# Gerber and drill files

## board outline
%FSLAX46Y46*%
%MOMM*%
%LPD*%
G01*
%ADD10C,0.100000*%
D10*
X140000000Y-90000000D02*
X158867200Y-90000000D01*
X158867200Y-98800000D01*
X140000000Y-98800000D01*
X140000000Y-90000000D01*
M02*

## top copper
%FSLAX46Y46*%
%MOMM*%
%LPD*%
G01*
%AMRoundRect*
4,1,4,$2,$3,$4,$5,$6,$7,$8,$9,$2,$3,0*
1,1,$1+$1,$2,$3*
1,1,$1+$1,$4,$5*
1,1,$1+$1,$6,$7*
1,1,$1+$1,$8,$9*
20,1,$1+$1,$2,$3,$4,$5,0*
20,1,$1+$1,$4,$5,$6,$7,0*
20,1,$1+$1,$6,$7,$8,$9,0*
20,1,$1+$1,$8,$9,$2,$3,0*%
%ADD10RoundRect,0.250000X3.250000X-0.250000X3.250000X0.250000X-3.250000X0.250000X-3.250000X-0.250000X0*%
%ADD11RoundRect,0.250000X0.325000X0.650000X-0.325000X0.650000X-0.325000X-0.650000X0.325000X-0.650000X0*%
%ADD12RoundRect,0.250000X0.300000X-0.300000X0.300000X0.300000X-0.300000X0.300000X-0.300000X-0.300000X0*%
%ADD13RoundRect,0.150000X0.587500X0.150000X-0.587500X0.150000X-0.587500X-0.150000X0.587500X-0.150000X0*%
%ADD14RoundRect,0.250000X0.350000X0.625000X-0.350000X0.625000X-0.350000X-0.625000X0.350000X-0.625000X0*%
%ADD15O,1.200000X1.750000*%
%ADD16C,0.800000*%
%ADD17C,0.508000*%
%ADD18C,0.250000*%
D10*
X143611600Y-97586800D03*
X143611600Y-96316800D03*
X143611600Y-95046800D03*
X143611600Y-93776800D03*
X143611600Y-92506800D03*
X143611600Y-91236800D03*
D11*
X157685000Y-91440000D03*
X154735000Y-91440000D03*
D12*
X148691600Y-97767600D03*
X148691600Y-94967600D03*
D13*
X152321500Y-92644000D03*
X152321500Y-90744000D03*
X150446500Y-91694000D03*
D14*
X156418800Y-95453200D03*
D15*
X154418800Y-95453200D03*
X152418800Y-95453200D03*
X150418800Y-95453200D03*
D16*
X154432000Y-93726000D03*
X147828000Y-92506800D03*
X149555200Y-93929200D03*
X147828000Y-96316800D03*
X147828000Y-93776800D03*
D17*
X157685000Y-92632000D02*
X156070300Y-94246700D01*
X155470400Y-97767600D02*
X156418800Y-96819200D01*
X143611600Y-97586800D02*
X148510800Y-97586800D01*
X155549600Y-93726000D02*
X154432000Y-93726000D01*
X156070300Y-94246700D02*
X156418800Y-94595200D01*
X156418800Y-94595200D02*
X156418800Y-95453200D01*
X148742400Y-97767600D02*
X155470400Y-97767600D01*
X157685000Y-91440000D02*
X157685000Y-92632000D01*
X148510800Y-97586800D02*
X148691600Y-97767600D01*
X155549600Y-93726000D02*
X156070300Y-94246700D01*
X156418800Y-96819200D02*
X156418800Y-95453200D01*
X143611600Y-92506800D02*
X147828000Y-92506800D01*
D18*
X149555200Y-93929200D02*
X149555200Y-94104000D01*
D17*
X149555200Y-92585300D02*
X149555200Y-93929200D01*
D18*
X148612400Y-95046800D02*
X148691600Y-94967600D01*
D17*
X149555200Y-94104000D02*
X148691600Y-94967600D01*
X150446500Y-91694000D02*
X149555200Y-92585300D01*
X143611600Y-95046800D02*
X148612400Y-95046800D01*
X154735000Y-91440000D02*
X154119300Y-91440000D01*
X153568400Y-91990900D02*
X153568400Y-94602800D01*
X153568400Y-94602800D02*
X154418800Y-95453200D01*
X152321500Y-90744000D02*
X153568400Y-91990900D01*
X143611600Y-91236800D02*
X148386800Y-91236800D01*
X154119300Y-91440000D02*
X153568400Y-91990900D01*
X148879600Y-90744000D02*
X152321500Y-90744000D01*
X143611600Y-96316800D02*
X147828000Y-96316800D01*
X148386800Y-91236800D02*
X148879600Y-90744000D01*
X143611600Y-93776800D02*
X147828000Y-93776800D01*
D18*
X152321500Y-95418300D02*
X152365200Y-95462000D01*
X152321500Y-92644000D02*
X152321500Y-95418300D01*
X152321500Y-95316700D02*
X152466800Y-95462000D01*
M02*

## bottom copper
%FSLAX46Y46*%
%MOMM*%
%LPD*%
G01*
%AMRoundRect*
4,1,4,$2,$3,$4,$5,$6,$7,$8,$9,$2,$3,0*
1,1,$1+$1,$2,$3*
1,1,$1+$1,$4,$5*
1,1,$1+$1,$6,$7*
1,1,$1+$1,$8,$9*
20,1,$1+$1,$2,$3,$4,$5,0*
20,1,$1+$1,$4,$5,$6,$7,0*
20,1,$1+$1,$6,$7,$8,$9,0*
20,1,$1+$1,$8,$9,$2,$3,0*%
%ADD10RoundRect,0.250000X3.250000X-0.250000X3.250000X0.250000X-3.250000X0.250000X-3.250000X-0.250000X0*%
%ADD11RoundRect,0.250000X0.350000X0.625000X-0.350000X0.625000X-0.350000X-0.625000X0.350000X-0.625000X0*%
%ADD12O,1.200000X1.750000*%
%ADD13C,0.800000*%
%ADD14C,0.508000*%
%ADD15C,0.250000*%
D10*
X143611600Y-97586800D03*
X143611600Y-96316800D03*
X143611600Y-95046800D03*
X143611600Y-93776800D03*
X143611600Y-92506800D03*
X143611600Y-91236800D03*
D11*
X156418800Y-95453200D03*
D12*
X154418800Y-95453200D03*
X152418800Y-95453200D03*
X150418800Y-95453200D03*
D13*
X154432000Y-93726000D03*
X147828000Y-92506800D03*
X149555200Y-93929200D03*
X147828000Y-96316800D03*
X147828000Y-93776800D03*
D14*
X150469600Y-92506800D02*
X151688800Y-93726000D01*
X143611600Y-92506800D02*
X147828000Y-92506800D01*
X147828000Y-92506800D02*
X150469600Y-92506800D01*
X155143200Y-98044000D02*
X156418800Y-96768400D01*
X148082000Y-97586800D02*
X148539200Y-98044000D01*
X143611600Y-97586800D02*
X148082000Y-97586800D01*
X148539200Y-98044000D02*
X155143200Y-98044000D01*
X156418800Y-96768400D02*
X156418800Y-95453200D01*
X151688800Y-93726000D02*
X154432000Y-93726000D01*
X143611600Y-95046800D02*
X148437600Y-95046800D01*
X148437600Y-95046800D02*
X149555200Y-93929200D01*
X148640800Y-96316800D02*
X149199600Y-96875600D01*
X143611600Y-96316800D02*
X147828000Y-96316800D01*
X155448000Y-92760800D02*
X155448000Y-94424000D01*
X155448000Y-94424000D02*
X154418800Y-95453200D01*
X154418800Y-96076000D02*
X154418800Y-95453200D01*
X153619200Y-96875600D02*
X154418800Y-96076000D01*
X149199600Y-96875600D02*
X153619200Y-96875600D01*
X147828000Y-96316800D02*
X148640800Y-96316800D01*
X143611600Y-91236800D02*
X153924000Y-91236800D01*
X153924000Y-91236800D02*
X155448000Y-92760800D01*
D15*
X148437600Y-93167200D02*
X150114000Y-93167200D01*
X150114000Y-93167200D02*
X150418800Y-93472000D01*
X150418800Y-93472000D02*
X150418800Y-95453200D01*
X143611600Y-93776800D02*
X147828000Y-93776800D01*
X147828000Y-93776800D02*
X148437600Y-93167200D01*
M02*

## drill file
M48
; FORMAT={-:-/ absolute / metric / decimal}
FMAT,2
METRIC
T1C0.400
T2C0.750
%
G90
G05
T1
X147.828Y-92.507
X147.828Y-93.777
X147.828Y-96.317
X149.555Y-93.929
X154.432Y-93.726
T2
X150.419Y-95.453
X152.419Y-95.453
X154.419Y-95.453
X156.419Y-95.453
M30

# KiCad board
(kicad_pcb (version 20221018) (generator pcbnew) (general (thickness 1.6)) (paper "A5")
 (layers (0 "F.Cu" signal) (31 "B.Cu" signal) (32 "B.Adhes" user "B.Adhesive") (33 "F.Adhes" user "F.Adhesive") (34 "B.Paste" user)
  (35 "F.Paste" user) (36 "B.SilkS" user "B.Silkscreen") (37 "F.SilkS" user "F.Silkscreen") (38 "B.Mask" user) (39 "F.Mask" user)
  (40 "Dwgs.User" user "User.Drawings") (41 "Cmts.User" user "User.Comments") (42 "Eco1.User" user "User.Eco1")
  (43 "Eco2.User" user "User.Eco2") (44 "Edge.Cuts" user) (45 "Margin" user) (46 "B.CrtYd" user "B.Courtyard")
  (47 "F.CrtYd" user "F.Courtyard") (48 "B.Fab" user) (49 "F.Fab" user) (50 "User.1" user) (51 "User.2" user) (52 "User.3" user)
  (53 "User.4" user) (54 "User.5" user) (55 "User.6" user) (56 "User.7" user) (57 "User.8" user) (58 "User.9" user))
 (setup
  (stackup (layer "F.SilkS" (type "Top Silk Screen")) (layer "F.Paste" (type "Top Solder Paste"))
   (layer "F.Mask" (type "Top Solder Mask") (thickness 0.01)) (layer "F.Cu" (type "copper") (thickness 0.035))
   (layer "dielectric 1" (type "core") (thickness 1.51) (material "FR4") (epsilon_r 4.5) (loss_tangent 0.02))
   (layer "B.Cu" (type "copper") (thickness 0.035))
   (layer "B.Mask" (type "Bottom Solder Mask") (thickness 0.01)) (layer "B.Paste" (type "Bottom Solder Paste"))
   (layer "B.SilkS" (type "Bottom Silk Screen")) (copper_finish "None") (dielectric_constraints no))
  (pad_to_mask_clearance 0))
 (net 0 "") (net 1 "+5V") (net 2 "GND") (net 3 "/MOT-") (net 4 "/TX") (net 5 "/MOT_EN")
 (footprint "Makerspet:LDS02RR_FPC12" (layer "F.Cu") (at 143.6116 94.4118 90)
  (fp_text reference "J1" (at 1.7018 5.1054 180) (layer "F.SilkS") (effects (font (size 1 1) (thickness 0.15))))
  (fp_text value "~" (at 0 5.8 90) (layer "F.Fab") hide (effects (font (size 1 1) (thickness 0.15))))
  (pad "1" smd roundrect (at -3.175 0 90) (size 1 7) (layers "F.Cu" "F.Mask") (roundrect_rratio 0.25) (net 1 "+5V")
   (thermal_bridge_angle 45))
  (pad "2" smd roundrect (at -3.175 0 90) (size 1 7) (layers "B.Cu" "B.Mask") (roundrect_rratio 0.25) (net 1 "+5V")
   (thermal_bridge_angle 45))
  (pad "3" smd roundrect (at -1.905 0 90) (size 1 7) (layers "F.Cu" "F.Mask") (roundrect_rratio 0.25) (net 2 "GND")
   (thermal_bridge_angle 45))
  (pad "4" smd roundrect (at -1.905 0 90) (size 1 7) (layers "B.Cu" "B.Mask") (roundrect_rratio 0.25) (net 2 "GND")
   (thermal_bridge_angle 45))
  (pad "5" smd roundrect (at -0.635 0 90) (size 1 7) (layers "F.Cu" "F.Mask") (roundrect_rratio 0.25) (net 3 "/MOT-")
   (thermal_bridge_angle 45))
  (pad "6" smd roundrect (at -0.635 0 90) (size 1 7) (layers "B.Cu" "B.Mask") (roundrect_rratio 0.25) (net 3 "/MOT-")
   (thermal_bridge_angle 45))
  (pad "7" smd roundrect (at 0.635 0 90) (size 1 7) (layers "F.Cu" "F.Mask") (roundrect_rratio 0.25) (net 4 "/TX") (thermal_bridge_angle 45))
  (pad "8" smd roundrect (at 0.635 0 90) (size 1 7) (layers "B.Cu" "B.Mask") (roundrect_rratio 0.25) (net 4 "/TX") (thermal_bridge_angle 45))
  (pad "9" smd roundrect (at 1.905 0 90) (size 1 7) (layers "F.Cu" "F.Mask") (roundrect_rratio 0.25) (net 1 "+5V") (thermal_bridge_angle 45))
  (pad "10" smd roundrect (at 1.905 0 90) (size 1 7) (layers "B.Cu" "B.Mask") (roundrect_rratio 0.25) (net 1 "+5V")
   (thermal_bridge_angle 45))
  (pad "11" smd roundrect (at 3.175 0 90) (size 1 7) (layers "F.Cu" "F.Mask") (roundrect_rratio 0.25) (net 2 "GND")
   (thermal_bridge_angle 45))
  (pad "12" smd roundrect (at 3.175 0 90) (size 1 7) (layers "B.Cu" "B.Mask") (roundrect_rratio 0.25) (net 2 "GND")
   (thermal_bridge_angle 45)))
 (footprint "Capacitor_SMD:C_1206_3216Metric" (layer "F.Cu") (at 156.21 91.44 180)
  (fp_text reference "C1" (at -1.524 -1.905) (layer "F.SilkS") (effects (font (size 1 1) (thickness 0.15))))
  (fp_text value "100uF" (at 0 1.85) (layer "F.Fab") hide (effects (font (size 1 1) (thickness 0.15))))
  (pad "1" smd roundrect (at -1.475 0 180) (size 1.15 1.8) (layers "F.Cu" "F.Paste" "F.Mask") (roundrect_rratio 0.2173913043) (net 1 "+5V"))
  (pad "2" smd roundrect (at 1.475 0 180) (size 1.15 1.8) (layers "F.Cu" "F.Paste" "F.Mask") (roundrect_rratio 0.2173913043) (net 2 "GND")))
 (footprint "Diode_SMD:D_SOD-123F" (layer "F.Cu") (at 148.6916 96.3676 90)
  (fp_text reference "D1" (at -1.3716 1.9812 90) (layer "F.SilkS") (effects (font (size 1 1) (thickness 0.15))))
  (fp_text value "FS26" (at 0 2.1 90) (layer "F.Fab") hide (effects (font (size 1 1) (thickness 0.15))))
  (pad "1" smd roundrect (at -1.4 0 90) (size 1.1 1.1) (layers "F.Cu" "F.Paste" "F.Mask") (roundrect_rratio 0.2272727273) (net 1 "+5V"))
  (pad "2" smd roundrect (at 1.4 0 90) (size 1.1 1.1) (layers "F.Cu" "F.Paste" "F.Mask") (roundrect_rratio 0.2272727273) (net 3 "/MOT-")))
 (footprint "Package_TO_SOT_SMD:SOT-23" (layer "F.Cu") (at 151.384 91.694 180)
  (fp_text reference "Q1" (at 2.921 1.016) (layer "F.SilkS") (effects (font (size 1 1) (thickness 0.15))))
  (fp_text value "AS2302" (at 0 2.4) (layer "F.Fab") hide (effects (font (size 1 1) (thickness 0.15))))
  (pad "1" smd roundrect (at -0.9375 -0.95 180) (size 1.475 0.6) (layers "F.Cu" "F.Paste" "F.Mask") (roundrect_rratio 0.25)
   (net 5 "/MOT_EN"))
  (pad "2" smd roundrect (at -0.9375 0.95 180) (size 1.475 0.6) (layers "F.Cu" "F.Paste" "F.Mask") (roundrect_rratio 0.25) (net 2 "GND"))
  (pad "3" smd roundrect (at 0.9375 0 180) (size 1.475 0.6) (layers "F.Cu" "F.Paste" "F.Mask") (roundrect_rratio 0.25) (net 3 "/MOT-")))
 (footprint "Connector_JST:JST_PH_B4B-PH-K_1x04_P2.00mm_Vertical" (layer "B.Cu") (at 156.4188 95.4532 180)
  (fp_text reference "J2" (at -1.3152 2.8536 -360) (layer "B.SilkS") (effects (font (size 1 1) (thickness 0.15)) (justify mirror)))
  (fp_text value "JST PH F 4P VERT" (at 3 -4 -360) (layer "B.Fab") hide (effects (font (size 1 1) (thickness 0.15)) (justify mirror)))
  (pad "1" thru_hole roundrect (at 0 0 180) (size 1.2 1.75) (drill 0.75) (layers "*.Cu" "*.Mask") (roundrect_rratio 0.2083333333)
   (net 1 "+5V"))
  (pad "2" thru_hole oval (at 2 0 180) (size 1.2 1.75) (drill 0.75) (layers "*.Cu" "*.Mask") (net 2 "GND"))
  (pad "3" thru_hole oval (at 4 0 180) (size 1.2 1.75) (drill 0.75) (layers "*.Cu" "*.Mask") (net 5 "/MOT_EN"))
  (pad "4" thru_hole oval (at 6 0 180) (size 1.2 1.75) (drill 0.75) (layers "*.Cu" "*.Mask") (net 4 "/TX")))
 (gr_rect (start 140 90) (end 158.8672 98.8) (stroke (width 0.1) (type default)) (fill none) (layer "Edge.Cuts"))
 (segment (start 157.685 92.632) (end 156.0703 94.2467) (width 0.508) (layer "F.Cu") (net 1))
 (segment (start 155.4704 97.7676) (end 156.4188 96.8192) (width 0.508) (layer "F.Cu") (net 1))
 (segment (start 143.6116 97.5868) (end 148.5108 97.5868) (width 0.508) (layer "F.Cu") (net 1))
 (segment (start 155.5496 93.726) (end 154.432 93.726) (width 0.508) (layer "F.Cu") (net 1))
 (segment (start 156.0703 94.2467) (end 156.4188 94.5952) (width 0.508) (layer "F.Cu") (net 1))
 (segment (start 156.4188 94.5952) (end 156.4188 95.4532) (width 0.508) (layer "F.Cu") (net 1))
 (segment (start 148.7424 97.7676) (end 155.4704 97.7676) (width 0.508) (layer "F.Cu") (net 1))
 (segment (start 157.685 91.44) (end 157.685 92.632) (width 0.508) (layer "F.Cu") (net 1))
 (segment (start 148.5108 97.5868) (end 148.6916 97.7676) (width 0.508) (layer "F.Cu") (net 1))
 (segment (start 155.5496 93.726) (end 156.0703 94.2467) (width 0.508) (layer "F.Cu") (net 1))
 (segment (start 156.4188 96.8192) (end 156.4188 95.4532) (width 0.508) (layer "F.Cu") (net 1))
 (segment (start 143.6116 92.5068) (end 147.828 92.5068) (width 0.508) (layer "F.Cu") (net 1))
 (via (at 154.432 93.726) (size 0.8) (drill 0.4) (layers "F.Cu" "B.Cu") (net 1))
 (via (at 147.828 92.5068) (size 0.8) (drill 0.4) (layers "F.Cu" "B.Cu") (free) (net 1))
 (segment (start 150.4696 92.5068) (end 151.6888 93.726) (width 0.508) (layer "B.Cu") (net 1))
 (segment (start 143.6116 92.5068) (end 147.828 92.5068) (width 0.508) (layer "B.Cu") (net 1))
 (segment (start 147.828 92.5068) (end 150.4696 92.5068) (width 0.508) (layer "B.Cu") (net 1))
 (segment (start 155.1432 98.044) (end 156.4188 96.7684) (width 0.508) (layer "B.Cu") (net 1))
 (segment (start 148.082 97.5868) (end 148.5392 98.044) (width 0.508) (layer "B.Cu") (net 1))
 (segment (start 143.6116 97.5868) (end 148.082 97.5868) (width 0.508) (layer "B.Cu") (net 1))
 (segment (start 148.5392 98.044) (end 155.1432 98.044) (width 0.508) (layer "B.Cu") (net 1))
 (segment (start 156.4188 96.7684) (end 156.4188 95.4532) (width 0.508) (layer "B.Cu") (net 1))
 (segment (start 151.6888 93.726) (end 154.432 93.726) (width 0.508) (layer "B.Cu") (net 1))
 (segment (start 149.5552 93.9292) (end 149.5552 94.104) (width 0.25) (layer "F.Cu") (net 3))
 (segment (start 149.5552 92.5853) (end 149.5552 93.9292) (width 0.508) (layer "F.Cu") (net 3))
 (segment (start 148.6124 95.0468) (end 148.6916 94.9676) (width 0.25) (layer "F.Cu") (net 3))
 (segment (start 149.5552 94.104) (end 148.6916 94.9676) (width 0.508) (layer "F.Cu") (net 3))
 (segment (start 150.4465 91.694) (end 149.5552 92.5853) (width 0.508) (layer "F.Cu") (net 3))
 (segment (start 143.6116 95.0468) (end 148.6124 95.0468) (width 0.508) (layer "F.Cu") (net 3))
 (via (at 149.5552 93.9292) (size 0.8) (drill 0.4) (layers "F.Cu" "B.Cu") (free) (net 3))
 (segment (start 143.6116 95.0468) (end 148.4376 95.0468) (width 0.508) (layer "B.Cu") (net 3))
 (segment (start 148.4376 95.0468) (end 149.5552 93.9292) (width 0.508) (layer "B.Cu") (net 3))
 (segment (start 154.735 91.44) (end 154.1193 91.44) (width 0.508) (layer "F.Cu") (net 2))
 (segment (start 153.5684 91.9909) (end 153.5684 94.6028) (width 0.508) (layer "F.Cu") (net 2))
 (segment (start 153.5684 94.6028) (end 154.4188 95.4532) (width 0.508) (layer "F.Cu") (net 2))
 (segment (start 152.3215 90.744) (end 153.5684 91.9909) (width 0.508) (layer "F.Cu") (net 2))
 (segment (start 143.6116 91.2368) (end 148.3868 91.2368) (width 0.508) (layer "F.Cu") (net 2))
 (segment (start 154.1193 91.44) (end 153.5684 91.9909) (width 0.508) (layer "F.Cu") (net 2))
 (segment (start 148.8796 90.744) (end 152.3215 90.744) (width 0.508) (layer "F.Cu") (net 2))
 (segment (start 143.6116 96.3168) (end 147.828 96.3168) (width 0.508) (layer "F.Cu") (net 2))
 (segment (start 148.3868 91.2368) (end 148.8796 90.744) (width 0.508) (layer "F.Cu") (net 2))
 (via (at 147.828 96.3168) (size 0.8) (drill 0.4) (layers "F.Cu" "B.Cu") (free) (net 2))
 (segment (start 148.6408 96.3168) (end 149.1996 96.8756) (width 0.508) (layer "B.Cu") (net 2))
 (segment (start 143.6116 96.3168) (end 147.828 96.3168) (width 0.508) (layer "B.Cu") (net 2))
 (segment (start 155.448 92.7608) (end 155.448 94.424) (width 0.508) (layer "B.Cu") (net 2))
 (segment (start 155.448 94.424) (end 154.4188 95.4532) (width 0.508) (layer "B.Cu") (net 2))
 (segment (start 154.4188 96.076) (end 154.4188 95.4532) (width 0.508) (layer "B.Cu") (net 2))
 (segment (start 153.6192 96.8756) (end 154.4188 96.076) (width 0.508) (layer "B.Cu") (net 2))
 (segment (start 149.1996 96.8756) (end 153.6192 96.8756) (width 0.508) (layer "B.Cu") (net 2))
 (segment (start 147.828 96.3168) (end 148.6408 96.3168) (width 0.508) (layer "B.Cu") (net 2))
 (segment (start 143.6116 91.2368) (end 153.924 91.2368) (width 0.508) (layer "B.Cu") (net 2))
 (segment (start 153.924 91.2368) (end 155.448 92.7608) (width 0.508) (layer "B.Cu") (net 2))
 (segment (start 143.6116 93.7768) (end 147.828 93.7768) (width 0.508) (layer "F.Cu") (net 4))
 (via (at 147.828 93.7768) (size 0.8) (drill 0.4) (layers "F.Cu" "B.Cu") (free) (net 4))
 (segment (start 148.4376 93.1672) (end 150.114 93.1672) (width 0.25) (layer "B.Cu") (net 4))
 (segment (start 150.114 93.1672) (end 150.4188 93.472) (width 0.25) (layer "B.Cu") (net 4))
 (segment (start 150.4188 93.472) (end 150.4188 95.4532) (width 0.25) (layer "B.Cu") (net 4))
 (segment (start 143.6116 93.7768) (end 147.828 93.7768) (width 0.25) (layer "B.Cu") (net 4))
 (segment (start 147.828 93.7768) (end 148.4376 93.1672) (width 0.25) (layer "B.Cu") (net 4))
 (segment (start 152.3215 95.4183) (end 152.3652 95.462) (width 0.25) (layer "F.Cu") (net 5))
 (segment (start 152.3215 92.644) (end 152.3215 95.4183) (width 0.25) (layer "F.Cu") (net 5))
 (segment (start 152.3215 95.3167) (end 152.4668 95.462) (width 0.25) (layer "F.Cu") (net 5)))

